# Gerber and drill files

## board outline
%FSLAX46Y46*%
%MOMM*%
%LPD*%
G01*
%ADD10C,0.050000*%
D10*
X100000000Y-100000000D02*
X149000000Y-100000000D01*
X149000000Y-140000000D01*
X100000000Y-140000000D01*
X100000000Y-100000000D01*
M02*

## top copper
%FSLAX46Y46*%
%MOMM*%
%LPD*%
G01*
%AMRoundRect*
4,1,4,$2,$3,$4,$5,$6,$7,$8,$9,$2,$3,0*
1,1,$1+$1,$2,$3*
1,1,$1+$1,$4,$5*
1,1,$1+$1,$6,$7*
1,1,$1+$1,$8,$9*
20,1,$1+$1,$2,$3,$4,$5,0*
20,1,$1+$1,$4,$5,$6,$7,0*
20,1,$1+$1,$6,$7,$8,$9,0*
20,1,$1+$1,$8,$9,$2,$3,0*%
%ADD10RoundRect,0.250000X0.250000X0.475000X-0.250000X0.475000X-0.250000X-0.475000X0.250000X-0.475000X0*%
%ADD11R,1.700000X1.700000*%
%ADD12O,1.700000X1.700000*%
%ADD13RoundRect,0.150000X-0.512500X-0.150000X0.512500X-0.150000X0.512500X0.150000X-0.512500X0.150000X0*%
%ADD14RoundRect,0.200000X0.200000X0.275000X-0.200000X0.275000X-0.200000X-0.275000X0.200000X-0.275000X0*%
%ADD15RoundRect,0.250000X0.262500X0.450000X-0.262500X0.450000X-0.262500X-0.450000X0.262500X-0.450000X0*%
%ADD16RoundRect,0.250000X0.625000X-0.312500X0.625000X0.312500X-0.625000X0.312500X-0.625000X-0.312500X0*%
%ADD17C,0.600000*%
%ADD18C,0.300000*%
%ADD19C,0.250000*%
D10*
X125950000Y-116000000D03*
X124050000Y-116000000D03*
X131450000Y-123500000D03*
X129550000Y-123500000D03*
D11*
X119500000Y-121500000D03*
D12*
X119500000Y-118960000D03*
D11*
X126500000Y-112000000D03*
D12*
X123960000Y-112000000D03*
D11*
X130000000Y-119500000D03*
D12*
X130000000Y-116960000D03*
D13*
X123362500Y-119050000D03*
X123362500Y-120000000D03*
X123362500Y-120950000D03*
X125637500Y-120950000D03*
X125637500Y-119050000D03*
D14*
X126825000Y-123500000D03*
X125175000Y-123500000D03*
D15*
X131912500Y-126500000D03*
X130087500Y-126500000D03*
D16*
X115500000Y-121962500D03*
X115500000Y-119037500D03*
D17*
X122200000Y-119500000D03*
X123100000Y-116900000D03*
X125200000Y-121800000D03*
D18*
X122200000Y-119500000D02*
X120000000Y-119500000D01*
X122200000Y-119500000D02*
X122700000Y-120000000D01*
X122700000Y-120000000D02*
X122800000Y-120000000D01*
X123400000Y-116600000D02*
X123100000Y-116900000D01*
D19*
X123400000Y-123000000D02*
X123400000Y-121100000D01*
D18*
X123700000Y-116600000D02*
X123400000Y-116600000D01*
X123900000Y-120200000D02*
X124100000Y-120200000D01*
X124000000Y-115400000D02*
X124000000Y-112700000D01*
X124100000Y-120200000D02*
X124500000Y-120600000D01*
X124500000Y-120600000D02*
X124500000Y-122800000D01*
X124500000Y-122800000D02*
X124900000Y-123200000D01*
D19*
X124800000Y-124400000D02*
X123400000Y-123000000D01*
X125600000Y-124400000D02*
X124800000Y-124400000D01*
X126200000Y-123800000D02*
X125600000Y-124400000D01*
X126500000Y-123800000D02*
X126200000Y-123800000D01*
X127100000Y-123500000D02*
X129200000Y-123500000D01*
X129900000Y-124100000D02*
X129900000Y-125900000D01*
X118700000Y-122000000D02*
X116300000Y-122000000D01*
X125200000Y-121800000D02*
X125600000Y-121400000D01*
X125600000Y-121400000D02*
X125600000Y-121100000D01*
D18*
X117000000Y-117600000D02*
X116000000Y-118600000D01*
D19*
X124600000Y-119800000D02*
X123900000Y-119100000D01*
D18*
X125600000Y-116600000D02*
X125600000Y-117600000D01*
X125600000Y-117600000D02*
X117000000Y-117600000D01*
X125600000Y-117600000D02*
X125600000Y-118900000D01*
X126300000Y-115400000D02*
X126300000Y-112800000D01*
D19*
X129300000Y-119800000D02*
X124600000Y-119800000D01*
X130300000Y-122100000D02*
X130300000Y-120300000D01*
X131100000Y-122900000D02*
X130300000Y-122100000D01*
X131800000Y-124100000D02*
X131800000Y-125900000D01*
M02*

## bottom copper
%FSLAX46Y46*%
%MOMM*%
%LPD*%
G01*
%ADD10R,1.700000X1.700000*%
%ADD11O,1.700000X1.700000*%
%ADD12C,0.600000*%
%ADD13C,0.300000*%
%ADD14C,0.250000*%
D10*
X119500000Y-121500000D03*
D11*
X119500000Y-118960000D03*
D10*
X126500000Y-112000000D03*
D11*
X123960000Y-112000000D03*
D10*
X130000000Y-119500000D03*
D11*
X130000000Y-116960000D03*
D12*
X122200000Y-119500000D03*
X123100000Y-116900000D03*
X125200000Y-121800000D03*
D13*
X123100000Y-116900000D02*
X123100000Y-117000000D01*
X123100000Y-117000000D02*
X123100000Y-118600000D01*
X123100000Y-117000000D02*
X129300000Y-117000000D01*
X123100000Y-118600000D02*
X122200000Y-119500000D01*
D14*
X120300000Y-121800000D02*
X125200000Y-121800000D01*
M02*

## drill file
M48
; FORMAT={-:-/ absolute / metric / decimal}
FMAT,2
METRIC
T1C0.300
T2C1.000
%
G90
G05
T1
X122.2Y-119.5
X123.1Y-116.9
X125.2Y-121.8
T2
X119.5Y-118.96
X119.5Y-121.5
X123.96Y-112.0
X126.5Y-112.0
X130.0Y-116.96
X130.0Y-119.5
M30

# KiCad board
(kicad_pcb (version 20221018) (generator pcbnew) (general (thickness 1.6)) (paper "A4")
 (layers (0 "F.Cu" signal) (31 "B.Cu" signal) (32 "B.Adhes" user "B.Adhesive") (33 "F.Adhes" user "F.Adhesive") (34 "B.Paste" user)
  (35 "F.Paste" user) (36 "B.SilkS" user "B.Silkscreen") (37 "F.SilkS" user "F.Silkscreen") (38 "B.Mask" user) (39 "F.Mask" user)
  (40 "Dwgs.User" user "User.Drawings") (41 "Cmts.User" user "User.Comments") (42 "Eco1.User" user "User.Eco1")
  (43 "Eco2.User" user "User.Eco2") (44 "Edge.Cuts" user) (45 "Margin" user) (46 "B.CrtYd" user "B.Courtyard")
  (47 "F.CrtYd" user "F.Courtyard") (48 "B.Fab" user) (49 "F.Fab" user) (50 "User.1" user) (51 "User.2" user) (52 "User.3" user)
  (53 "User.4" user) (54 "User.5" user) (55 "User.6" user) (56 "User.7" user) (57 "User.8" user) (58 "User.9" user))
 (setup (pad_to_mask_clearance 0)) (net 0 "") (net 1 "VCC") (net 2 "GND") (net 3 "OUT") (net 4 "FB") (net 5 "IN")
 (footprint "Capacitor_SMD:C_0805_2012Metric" (layer "F.Cu") (at 125 116 180)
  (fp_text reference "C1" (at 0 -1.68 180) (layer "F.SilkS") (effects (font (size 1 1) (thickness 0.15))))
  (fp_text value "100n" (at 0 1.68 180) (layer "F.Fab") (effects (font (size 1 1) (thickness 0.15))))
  (pad "1" smd roundrect (at -0.95 0 180) (size 1 1.45) (layers "F.Cu" "F.Paste" "F.Mask") (roundrect_rratio 0.25) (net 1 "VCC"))
  (pad "2" smd roundrect (at 0.95 0 180) (size 1 1.45) (layers "F.Cu" "F.Paste" "F.Mask") (roundrect_rratio 0.25) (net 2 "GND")))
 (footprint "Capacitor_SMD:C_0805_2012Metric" (layer "F.Cu") (at 130.5 123.5 180)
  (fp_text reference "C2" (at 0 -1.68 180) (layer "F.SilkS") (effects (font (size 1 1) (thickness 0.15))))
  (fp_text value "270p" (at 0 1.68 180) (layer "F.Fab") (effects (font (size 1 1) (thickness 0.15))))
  (pad "1" smd roundrect (at -0.95 0 180) (size 1 1.45) (layers "F.Cu" "F.Paste" "F.Mask") (roundrect_rratio 0.25) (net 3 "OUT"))
  (pad "2" smd roundrect (at 0.95 0 180) (size 1 1.45) (layers "F.Cu" "F.Paste" "F.Mask") (roundrect_rratio 0.25) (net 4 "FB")))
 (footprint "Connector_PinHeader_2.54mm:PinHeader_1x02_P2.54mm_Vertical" (layer "F.Cu") (at 119.5 121.5 180)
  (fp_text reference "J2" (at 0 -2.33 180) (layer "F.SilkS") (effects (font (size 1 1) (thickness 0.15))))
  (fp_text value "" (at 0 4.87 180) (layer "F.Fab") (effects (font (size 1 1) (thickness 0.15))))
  (pad "1" thru_hole rect (at 0 0 180) (size 1.7 1.7) (drill 1) (layers "*.Cu" "*.Mask") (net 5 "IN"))
  (pad "2" thru_hole oval (at 0 2.54 180) (size 1.7 1.7) (drill 1) (layers "*.Cu" "*.Mask") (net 2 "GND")))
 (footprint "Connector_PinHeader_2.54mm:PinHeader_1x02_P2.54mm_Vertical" (layer "F.Cu") (at 126.5 112 -90)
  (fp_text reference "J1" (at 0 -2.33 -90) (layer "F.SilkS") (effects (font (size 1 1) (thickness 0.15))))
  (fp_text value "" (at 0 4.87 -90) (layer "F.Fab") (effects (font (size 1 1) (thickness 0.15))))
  (pad "1" thru_hole rect (at 0 0 270) (size 1.7 1.7) (drill 1) (layers "*.Cu" "*.Mask") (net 1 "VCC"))
  (pad "2" thru_hole oval (at 0 2.54 270) (size 1.7 1.7) (drill 1) (layers "*.Cu" "*.Mask") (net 2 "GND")))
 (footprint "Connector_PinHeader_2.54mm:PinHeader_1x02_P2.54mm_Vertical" (layer "F.Cu") (at 130 119.5 180)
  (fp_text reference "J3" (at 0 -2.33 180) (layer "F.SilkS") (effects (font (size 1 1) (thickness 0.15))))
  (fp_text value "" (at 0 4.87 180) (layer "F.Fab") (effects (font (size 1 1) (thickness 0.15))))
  (pad "1" thru_hole rect (at 0 0 180) (size 1.7 1.7) (drill 1) (layers "*.Cu" "*.Mask") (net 3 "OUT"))
  (pad "2" thru_hole oval (at 0 2.54 180) (size 1.7 1.7) (drill 1) (layers "*.Cu" "*.Mask") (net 2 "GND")))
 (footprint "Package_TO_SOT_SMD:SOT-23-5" (layer "F.Cu") (at 124.5 120)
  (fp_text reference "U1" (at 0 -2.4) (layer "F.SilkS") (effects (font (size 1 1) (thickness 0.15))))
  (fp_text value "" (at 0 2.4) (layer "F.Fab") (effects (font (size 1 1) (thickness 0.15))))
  (pad "1" smd roundrect (at -1.1375 -0.95) (size 1.325 0.6) (layers "F.Cu" "F.Paste" "F.Mask") (roundrect_rratio 0.25) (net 3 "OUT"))
  (pad "2" smd roundrect (at -1.1375 0) (size 1.325 0.6) (layers "F.Cu" "F.Paste" "F.Mask") (roundrect_rratio 0.25) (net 2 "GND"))
  (pad "3" smd roundrect (at -1.1375 0.95) (size 1.325 0.6) (layers "F.Cu" "F.Paste" "F.Mask") (roundrect_rratio 0.25) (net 4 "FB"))
  (pad "4" smd roundrect (at 1.1375 0.95) (size 1.325 0.6) (layers "F.Cu" "F.Paste" "F.Mask") (roundrect_rratio 0.25) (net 5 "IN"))
  (pad "5" smd roundrect (at 1.1375 -0.95) (size 1.325 0.6) (layers "F.Cu" "F.Paste" "F.Mask") (roundrect_rratio 0.25) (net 1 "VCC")))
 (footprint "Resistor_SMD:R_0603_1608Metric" (layer "F.Cu") (at 126 123.5 180)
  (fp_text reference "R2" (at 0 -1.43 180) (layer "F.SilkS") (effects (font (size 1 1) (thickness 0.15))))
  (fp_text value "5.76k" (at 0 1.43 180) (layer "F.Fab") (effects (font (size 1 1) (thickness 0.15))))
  (pad "1" smd roundrect (at -0.825 0 180) (size 0.8 0.95) (layers "F.Cu" "F.Paste" "F.Mask") (roundrect_rratio 0.25) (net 4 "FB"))
  (pad "2" smd roundrect (at 0.825 0 180) (size 0.8 0.95) (layers "F.Cu" "F.Paste" "F.Mask") (roundrect_rratio 0.25) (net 2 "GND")))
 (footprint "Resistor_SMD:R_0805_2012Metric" (layer "F.Cu") (at 131 126.5 180)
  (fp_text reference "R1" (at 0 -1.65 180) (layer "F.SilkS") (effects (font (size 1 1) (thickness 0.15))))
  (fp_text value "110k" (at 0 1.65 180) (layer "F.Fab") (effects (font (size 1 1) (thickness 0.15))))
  (pad "1" smd roundrect (at -0.9125 0 180) (size 1.025 1.4) (layers "F.Cu" "F.Paste" "F.Mask") (roundrect_rratio 0.243902) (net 3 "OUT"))
  (pad "2" smd roundrect (at 0.9125 0 180) (size 1.025 1.4) (layers "F.Cu" "F.Paste" "F.Mask") (roundrect_rratio 0.243902) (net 4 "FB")))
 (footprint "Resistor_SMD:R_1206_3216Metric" (layer "F.Cu") (at 115.5 120.5 90)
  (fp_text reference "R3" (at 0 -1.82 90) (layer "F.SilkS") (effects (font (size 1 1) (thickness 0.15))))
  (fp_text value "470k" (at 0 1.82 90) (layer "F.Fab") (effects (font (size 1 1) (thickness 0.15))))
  (pad "1" smd roundrect (at -1.4625 0 90) (size 1.125 1.75) (layers "F.Cu" "F.Paste" "F.Mask") (roundrect_rratio 0.222222) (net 5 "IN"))
  (pad "2" smd roundrect (at 1.4625 0 90) (size 1.125 1.75) (layers "F.Cu" "F.Paste" "F.Mask") (roundrect_rratio 0.222222) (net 1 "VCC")))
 (gr_rect (start 100 100) (end 149 140) (stroke (width 0.05) (type default)) (fill none) (layer "Edge.Cuts"))
 (segment (start 122.2 119.5) (end 120 119.5) (width 0.3) (layer "F.Cu") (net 2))
 (segment (start 122.2 119.5) (end 122.7 120) (width 0.3) (layer "F.Cu") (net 2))
 (segment (start 122.7 120) (end 122.8 120) (width 0.3) (layer "F.Cu") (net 2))
 (segment (start 123.4 116.6) (end 123.1 116.9) (width 0.3) (layer "F.Cu") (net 2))
 (segment (start 123.4 123) (end 123.4 121.1) (width 0.25) (layer "F.Cu") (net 4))
 (segment (start 123.7 116.6) (end 123.4 116.6) (width 0.3) (layer "F.Cu") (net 2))
 (segment (start 123.9 120.2) (end 124.1 120.2) (width 0.3) (layer "F.Cu") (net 2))
 (segment (start 124 115.4) (end 124 112.7) (width 0.3) (layer "F.Cu") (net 2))
 (segment (start 124.1 120.2) (end 124.5 120.6) (width 0.3) (layer "F.Cu") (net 2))
 (segment (start 124.5 120.6) (end 124.5 122.8) (width 0.3) (layer "F.Cu") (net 2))
 (segment (start 124.5 122.8) (end 124.9 123.2) (width 0.3) (layer "F.Cu") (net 2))
 (segment (start 124.8 124.4) (end 123.4 123) (width 0.25) (layer "F.Cu") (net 4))
 (segment (start 125.6 124.4) (end 124.8 124.4) (width 0.25) (layer "F.Cu") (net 4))
 (segment (start 126.2 123.8) (end 125.6 124.4) (width 0.25) (layer "F.Cu") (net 4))
 (segment (start 126.5 123.8) (end 126.2 123.8) (width 0.25) (layer "F.Cu") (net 4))
 (segment (start 127.1 123.5) (end 129.2 123.5) (width 0.25) (layer "F.Cu") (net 4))
 (segment (start 129.9 124.1) (end 129.9 125.9) (width 0.25) (layer "F.Cu") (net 4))
 (via (at 122.2 119.5) (size 0.6) (drill 0.3) (layers "F.Cu" "B.Cu") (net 2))
 (via (at 123.1 116.9) (size 0.6) (drill 0.3) (layers "F.Cu" "B.Cu") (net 2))
 (segment (start 118.7 122) (end 116.3 122) (width 0.25) (layer "F.Cu") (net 5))
 (segment (start 123.1 116.9) (end 123.1 117) (width 0.3) (layer "B.Cu") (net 2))
 (segment (start 123.1 117) (end 123.1 118.6) (width 0.3) (layer "B.Cu") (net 2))
 (segment (start 123.1 117) (end 129.3 117) (width 0.3) (layer "B.Cu") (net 2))
 (segment (start 123.1 118.6) (end 122.2 119.5) (width 0.3) (layer "B.Cu") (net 2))
 (segment (start 125.2 121.8) (end 125.6 121.4) (width 0.25) (layer "F.Cu") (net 5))
 (segment (start 125.6 121.4) (end 125.6 121.1) (width 0.25) (layer "F.Cu") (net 5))
 (via (at 125.2 121.8) (size 0.6) (drill 0.3) (layers "F.Cu" "B.Cu") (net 5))
 (segment (start 117 117.6) (end 116 118.6) (width 0.3) (layer "F.Cu") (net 1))
 (segment (start 120.3 121.8) (end 125.2 121.8) (width 0.25) (layer "B.Cu") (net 5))
 (segment (start 124.6 119.8) (end 123.9 119.1) (width 0.25) (layer "F.Cu") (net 3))
 (segment (start 125.6 116.6) (end 125.6 117.6) (width 0.3) (layer "F.Cu") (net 1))
 (segment (start 125.6 117.6) (end 117 117.6) (width 0.3) (layer "F.Cu") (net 1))
 (segment (start 125.6 117.6) (end 125.6 118.9) (width 0.3) (layer "F.Cu") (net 1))
 (segment (start 126.3 115.4) (end 126.3 112.8) (width 0.3) (layer "F.Cu") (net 1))
 (segment (start 129.3 119.8) (end 124.6 119.8) (width 0.25) (layer "F.Cu") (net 3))
 (segment (start 130.3 122.1) (end 130.3 120.3) (width 0.25) (layer "F.Cu") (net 3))
 (segment (start 131.1 122.9) (end 130.3 122.1) (width 0.25) (layer "F.Cu") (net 3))
 (segment (start 131.8 124.1) (end 131.8 125.9) (width 0.25) (layer "F.Cu") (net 3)))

